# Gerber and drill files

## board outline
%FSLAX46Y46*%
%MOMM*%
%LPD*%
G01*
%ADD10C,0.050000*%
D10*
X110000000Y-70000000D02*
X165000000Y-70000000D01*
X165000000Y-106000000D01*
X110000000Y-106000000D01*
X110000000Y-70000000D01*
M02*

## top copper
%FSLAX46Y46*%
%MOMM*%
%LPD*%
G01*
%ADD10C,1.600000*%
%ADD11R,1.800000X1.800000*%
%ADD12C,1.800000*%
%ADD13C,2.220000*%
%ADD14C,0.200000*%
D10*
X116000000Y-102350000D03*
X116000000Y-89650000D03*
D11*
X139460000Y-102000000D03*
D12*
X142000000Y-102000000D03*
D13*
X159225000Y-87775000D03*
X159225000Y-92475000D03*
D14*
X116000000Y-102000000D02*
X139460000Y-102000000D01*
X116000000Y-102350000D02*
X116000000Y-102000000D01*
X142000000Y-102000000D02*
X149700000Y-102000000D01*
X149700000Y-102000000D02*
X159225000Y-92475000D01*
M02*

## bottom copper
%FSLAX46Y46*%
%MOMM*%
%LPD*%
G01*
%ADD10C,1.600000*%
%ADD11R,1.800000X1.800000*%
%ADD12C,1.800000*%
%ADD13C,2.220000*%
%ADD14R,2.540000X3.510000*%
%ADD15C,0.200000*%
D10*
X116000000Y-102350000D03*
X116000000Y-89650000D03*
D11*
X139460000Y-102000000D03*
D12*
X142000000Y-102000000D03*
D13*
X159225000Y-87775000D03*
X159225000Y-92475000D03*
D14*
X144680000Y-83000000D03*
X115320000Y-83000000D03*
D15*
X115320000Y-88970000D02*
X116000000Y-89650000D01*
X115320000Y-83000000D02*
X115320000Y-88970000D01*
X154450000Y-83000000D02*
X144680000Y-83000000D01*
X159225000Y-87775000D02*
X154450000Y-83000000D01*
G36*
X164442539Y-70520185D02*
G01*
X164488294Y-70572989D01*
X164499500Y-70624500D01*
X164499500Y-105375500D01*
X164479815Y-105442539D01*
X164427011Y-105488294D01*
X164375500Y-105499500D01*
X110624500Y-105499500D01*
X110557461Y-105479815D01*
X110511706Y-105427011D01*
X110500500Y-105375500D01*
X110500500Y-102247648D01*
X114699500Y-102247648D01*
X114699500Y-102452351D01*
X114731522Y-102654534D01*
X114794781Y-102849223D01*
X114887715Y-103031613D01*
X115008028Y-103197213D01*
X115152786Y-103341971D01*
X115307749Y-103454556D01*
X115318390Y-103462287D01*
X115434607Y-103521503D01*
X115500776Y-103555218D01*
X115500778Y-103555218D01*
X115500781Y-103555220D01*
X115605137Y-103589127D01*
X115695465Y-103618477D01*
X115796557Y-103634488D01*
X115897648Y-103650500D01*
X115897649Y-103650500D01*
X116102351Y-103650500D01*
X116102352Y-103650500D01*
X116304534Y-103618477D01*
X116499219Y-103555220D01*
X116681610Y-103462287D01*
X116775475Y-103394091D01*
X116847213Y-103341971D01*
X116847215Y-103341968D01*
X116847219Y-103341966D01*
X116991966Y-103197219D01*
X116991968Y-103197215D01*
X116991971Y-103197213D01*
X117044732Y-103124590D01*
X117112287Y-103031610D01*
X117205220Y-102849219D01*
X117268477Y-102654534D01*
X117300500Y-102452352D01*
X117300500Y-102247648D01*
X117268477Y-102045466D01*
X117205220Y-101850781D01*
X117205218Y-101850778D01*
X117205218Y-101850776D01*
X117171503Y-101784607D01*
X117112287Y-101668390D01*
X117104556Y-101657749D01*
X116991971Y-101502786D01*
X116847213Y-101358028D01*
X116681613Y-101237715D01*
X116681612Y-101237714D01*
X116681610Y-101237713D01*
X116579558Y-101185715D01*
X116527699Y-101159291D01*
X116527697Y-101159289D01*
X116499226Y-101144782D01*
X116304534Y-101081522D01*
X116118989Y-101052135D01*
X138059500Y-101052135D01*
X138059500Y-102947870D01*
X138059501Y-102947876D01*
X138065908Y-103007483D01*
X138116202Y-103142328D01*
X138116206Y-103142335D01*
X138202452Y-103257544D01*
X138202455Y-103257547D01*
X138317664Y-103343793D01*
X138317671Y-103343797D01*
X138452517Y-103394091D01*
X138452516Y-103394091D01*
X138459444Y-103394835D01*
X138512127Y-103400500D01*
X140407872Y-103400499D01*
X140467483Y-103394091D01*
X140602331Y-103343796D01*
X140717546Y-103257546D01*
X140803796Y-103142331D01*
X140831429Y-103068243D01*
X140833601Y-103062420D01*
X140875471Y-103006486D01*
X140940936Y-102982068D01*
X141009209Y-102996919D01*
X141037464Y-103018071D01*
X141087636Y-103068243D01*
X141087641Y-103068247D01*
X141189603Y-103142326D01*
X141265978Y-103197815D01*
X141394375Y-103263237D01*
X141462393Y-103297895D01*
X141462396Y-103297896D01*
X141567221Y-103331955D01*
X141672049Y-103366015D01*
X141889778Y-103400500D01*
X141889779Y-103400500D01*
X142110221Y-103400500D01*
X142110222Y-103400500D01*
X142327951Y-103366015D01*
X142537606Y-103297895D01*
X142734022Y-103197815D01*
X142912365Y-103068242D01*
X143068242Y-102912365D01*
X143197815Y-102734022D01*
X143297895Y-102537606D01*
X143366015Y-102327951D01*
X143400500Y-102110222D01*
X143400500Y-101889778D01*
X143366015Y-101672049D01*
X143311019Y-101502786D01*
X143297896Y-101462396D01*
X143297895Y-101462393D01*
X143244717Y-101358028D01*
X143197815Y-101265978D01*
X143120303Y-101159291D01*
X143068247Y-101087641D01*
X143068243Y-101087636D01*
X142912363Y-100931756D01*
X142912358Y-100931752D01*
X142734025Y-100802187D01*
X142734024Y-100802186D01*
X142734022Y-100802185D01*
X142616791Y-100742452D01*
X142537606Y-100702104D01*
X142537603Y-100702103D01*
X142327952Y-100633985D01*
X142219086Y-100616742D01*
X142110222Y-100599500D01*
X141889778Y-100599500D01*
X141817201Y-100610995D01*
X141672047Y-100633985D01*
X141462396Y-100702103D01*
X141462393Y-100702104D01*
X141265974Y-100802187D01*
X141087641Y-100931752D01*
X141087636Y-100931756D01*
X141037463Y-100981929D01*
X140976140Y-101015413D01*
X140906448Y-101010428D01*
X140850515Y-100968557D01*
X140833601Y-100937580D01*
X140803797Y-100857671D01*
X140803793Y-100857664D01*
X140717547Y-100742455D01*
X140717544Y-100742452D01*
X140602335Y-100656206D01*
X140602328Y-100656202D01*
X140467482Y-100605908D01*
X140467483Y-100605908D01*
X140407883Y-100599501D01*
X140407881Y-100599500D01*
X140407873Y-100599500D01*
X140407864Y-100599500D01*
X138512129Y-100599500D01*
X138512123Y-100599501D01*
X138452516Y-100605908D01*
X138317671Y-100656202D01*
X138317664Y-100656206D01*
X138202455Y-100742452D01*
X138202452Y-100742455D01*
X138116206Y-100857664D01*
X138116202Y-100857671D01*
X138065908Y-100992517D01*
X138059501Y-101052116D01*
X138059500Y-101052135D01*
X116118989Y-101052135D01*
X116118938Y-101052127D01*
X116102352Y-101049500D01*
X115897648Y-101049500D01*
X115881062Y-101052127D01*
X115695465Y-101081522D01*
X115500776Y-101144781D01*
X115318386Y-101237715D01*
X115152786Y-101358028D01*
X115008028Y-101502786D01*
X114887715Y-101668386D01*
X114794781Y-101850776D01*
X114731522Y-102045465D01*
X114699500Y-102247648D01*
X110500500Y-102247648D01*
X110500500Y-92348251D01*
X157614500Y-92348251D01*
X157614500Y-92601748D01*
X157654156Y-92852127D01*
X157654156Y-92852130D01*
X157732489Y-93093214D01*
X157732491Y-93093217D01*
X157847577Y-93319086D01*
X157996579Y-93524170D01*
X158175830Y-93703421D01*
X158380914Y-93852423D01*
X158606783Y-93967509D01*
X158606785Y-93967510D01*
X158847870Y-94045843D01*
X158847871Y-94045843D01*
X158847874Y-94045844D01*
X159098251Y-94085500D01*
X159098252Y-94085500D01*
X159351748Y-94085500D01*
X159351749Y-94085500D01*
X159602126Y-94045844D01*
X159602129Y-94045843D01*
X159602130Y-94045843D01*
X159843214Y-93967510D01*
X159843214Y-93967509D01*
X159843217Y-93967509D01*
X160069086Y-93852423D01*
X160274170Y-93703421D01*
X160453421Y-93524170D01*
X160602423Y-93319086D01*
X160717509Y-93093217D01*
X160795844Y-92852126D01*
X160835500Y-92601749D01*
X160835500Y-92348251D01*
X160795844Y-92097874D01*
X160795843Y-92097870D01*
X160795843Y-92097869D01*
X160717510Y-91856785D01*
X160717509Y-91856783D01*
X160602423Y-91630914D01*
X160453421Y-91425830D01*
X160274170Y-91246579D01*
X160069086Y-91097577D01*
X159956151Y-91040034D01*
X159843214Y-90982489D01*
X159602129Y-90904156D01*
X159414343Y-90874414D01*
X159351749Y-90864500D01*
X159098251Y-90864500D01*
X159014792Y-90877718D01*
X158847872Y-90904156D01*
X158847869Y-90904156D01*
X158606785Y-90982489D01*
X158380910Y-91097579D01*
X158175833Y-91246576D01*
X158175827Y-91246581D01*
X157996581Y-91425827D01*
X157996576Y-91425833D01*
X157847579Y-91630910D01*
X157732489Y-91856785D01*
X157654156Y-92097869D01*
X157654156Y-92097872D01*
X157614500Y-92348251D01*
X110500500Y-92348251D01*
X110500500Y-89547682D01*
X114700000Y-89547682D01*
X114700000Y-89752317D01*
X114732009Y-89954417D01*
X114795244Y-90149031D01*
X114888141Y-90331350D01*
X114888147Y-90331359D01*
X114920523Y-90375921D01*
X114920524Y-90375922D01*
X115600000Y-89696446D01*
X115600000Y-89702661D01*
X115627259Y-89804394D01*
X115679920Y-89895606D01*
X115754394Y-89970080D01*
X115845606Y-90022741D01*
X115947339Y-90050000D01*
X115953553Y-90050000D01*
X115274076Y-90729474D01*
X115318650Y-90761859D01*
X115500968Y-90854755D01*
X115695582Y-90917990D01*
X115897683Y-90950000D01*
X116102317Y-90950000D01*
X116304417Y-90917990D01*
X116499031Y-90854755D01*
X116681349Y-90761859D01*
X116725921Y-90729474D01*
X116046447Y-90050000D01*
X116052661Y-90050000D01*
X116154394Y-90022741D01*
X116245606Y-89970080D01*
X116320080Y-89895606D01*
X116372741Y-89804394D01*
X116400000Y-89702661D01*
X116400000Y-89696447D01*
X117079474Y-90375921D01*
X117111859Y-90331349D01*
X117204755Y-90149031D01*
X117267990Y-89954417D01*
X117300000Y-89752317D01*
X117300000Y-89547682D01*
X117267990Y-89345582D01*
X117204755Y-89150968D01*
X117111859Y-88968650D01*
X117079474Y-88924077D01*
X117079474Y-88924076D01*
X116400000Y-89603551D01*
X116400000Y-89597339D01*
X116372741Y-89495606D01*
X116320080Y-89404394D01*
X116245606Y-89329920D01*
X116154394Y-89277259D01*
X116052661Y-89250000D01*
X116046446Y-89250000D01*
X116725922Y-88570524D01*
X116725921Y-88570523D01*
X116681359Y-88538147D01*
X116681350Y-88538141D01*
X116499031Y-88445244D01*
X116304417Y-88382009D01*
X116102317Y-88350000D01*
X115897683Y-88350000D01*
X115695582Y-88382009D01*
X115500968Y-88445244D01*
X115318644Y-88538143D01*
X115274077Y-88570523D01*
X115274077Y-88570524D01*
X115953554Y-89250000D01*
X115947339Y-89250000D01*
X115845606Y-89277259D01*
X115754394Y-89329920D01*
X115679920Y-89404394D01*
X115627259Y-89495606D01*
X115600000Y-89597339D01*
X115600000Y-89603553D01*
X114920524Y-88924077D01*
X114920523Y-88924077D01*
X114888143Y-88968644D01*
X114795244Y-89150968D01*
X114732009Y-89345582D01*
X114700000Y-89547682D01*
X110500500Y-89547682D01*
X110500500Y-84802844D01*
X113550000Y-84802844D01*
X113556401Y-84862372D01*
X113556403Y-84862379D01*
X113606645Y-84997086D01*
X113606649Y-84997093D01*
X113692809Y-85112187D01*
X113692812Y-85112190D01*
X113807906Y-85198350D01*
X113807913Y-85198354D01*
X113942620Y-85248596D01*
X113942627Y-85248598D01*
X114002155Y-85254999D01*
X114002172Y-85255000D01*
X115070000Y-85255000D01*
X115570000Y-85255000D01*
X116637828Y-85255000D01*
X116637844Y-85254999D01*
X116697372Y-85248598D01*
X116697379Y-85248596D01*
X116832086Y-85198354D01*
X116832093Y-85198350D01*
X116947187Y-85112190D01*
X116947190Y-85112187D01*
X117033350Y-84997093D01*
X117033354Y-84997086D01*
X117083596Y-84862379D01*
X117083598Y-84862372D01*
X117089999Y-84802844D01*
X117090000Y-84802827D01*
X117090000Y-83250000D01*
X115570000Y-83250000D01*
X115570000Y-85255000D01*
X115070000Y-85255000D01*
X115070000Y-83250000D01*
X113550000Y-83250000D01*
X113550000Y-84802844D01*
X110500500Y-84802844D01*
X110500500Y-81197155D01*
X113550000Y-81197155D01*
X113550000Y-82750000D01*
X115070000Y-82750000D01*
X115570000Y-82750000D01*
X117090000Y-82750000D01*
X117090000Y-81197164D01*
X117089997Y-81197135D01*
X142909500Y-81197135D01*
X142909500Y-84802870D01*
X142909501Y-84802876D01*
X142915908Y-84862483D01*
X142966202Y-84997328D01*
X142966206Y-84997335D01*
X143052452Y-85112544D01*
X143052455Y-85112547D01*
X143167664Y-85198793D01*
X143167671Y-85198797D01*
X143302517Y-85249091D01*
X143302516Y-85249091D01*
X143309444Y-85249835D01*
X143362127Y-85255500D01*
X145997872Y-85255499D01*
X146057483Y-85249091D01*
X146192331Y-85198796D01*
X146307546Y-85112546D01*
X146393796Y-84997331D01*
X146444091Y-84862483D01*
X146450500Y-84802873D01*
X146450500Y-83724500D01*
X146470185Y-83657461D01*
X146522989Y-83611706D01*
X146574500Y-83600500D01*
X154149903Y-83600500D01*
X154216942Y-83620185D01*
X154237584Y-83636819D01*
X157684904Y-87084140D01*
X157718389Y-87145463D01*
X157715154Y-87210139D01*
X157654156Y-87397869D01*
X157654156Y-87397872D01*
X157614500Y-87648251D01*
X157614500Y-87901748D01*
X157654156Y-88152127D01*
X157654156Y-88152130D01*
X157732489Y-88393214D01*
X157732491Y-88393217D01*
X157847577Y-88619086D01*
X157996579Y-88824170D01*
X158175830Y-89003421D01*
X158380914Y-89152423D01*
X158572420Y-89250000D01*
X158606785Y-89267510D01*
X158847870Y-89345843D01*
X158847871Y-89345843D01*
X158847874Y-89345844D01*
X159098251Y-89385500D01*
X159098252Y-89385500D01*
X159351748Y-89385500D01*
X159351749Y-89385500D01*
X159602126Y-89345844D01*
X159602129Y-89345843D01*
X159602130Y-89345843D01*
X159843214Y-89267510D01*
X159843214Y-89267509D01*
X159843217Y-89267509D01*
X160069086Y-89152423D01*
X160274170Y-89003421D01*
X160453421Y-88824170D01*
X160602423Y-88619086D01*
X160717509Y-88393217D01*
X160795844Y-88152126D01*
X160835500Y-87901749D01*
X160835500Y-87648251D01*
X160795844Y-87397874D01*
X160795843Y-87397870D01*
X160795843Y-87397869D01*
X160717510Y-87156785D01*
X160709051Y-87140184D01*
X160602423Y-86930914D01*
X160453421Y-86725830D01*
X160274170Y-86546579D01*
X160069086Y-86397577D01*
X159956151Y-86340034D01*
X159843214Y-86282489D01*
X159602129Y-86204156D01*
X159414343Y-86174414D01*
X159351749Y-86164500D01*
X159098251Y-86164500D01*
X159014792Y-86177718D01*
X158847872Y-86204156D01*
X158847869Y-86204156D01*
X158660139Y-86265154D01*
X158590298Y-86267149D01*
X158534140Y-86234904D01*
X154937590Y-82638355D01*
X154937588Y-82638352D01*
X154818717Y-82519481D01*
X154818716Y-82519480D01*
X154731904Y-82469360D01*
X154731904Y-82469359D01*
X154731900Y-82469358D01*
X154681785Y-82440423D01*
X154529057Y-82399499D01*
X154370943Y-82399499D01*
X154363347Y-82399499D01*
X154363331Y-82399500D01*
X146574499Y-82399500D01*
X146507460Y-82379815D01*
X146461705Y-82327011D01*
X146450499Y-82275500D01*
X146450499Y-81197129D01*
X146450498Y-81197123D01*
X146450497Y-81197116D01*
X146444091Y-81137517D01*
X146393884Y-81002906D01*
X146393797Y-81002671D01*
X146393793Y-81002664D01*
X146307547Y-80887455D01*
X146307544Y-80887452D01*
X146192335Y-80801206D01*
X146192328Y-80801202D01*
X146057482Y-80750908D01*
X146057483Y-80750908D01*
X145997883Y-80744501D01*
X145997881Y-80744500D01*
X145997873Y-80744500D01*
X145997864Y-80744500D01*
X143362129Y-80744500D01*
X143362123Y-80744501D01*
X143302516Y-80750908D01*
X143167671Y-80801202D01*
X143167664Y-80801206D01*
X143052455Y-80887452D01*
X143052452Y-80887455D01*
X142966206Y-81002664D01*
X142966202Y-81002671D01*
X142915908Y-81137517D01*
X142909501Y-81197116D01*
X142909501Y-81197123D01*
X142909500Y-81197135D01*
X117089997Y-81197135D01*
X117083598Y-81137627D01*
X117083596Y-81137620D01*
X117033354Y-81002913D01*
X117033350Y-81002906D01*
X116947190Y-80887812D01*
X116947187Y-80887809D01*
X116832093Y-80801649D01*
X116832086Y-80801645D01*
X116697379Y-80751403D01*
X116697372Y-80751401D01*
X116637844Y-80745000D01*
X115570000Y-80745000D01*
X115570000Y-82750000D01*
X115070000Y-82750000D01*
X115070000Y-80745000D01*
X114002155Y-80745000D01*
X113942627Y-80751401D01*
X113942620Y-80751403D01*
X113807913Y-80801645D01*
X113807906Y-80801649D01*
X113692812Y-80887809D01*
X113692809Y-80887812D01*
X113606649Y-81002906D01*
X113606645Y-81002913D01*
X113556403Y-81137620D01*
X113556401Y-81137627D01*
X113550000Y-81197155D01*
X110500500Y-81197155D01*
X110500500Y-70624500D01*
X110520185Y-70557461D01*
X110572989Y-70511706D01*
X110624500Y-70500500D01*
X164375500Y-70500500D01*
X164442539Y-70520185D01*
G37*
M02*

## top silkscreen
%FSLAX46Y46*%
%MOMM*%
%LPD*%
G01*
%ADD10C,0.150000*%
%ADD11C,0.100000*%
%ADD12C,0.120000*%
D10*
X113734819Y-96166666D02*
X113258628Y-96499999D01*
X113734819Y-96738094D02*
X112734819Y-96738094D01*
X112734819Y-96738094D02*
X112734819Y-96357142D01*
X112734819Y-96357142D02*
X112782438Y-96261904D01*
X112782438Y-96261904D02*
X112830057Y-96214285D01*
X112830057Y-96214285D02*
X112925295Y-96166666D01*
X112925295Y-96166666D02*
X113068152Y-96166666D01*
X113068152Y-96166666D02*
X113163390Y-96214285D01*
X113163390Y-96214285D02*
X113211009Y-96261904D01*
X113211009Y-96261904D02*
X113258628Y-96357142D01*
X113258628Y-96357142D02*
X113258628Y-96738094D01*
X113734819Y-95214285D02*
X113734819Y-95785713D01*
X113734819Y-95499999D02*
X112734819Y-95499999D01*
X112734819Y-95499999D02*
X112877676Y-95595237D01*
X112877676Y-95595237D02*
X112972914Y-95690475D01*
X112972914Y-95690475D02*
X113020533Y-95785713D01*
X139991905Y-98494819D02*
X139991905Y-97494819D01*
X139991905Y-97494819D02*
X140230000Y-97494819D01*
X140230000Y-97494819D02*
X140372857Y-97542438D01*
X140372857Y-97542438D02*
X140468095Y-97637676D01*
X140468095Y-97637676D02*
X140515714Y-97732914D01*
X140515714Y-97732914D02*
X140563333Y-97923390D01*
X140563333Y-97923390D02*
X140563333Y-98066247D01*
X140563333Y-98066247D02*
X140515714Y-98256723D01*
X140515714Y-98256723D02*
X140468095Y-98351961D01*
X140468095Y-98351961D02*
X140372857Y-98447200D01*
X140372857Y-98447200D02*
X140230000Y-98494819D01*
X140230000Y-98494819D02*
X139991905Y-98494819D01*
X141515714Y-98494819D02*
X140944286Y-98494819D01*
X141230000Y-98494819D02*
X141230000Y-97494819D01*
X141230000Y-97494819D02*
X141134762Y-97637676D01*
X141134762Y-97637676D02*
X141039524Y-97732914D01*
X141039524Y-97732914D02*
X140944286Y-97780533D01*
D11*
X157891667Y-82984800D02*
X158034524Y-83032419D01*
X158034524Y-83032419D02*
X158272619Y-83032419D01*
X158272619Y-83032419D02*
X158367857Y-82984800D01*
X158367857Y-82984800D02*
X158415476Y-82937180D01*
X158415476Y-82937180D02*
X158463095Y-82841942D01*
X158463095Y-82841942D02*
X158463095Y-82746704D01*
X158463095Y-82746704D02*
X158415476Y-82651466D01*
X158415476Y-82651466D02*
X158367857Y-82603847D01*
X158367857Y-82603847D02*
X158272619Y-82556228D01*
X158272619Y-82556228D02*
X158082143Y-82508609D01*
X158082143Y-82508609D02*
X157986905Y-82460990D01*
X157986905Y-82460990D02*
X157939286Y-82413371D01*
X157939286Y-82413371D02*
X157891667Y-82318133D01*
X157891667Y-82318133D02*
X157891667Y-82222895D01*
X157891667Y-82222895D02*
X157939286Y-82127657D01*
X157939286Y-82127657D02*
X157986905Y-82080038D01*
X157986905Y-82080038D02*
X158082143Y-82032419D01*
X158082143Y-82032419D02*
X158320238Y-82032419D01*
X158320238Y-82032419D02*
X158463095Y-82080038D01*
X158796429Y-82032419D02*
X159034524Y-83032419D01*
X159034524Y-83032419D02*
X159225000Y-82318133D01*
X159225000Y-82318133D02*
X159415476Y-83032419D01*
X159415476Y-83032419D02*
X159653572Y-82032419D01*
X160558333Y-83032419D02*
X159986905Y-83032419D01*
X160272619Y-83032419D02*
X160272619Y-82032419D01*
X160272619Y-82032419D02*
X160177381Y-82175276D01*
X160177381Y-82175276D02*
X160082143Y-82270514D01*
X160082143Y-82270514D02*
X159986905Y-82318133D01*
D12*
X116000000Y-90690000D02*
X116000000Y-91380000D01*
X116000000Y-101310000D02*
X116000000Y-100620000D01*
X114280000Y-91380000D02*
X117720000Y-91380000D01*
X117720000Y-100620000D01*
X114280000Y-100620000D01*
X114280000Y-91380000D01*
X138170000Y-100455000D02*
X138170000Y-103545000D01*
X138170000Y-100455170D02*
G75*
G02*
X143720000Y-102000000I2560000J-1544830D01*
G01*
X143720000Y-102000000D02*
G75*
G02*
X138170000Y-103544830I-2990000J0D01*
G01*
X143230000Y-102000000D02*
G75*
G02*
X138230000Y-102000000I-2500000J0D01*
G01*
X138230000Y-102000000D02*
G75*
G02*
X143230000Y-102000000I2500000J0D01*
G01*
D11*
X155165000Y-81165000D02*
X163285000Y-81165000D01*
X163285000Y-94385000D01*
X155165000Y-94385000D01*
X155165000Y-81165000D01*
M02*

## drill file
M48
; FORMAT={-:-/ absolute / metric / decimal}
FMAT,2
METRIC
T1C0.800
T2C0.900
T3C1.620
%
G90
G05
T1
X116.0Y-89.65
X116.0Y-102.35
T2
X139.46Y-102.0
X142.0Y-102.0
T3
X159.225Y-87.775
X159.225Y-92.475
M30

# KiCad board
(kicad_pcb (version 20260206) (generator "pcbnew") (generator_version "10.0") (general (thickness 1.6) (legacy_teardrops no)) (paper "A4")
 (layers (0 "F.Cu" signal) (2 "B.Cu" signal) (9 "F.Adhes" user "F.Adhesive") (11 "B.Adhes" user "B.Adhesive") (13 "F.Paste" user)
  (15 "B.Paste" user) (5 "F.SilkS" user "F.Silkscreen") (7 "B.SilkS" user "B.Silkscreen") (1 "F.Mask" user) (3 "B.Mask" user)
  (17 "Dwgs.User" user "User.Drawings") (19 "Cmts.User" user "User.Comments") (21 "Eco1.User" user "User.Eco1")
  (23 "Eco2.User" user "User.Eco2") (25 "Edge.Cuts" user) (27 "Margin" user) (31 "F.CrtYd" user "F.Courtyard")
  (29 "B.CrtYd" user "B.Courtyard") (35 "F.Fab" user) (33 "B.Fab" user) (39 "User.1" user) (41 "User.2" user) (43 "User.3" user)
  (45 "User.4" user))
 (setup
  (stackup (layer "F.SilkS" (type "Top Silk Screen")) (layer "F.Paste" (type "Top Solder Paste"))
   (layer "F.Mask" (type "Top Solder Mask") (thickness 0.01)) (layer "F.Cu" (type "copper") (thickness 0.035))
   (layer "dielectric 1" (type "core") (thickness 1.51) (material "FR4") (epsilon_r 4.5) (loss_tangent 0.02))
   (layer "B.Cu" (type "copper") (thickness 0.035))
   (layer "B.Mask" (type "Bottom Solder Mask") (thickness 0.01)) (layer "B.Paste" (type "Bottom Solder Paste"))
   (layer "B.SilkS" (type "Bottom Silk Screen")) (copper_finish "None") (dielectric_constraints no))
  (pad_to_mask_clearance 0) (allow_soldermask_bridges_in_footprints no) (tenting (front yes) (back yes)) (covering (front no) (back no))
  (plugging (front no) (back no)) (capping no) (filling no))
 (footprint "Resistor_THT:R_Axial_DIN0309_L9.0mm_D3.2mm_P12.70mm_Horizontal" (layer "F.Cu") (at 116 102.35 90)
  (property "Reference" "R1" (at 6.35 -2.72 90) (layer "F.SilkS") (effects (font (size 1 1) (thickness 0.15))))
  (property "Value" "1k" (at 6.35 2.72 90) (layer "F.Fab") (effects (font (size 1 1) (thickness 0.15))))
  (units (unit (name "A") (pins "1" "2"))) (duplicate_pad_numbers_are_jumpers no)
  (fp_line (start 11.66 0) (end 10.97 0) (stroke (width 0.12) (type solid)) (layer "F.SilkS"))
  (fp_line (start 1.04 0) (end 1.73 0) (stroke (width 0.12) (type solid)) (layer "F.SilkS"))
  (fp_rect (start 1.73 -1.72) (end 10.97 1.72) (stroke (width 0.12) (type solid)) (fill no) (layer "F.SilkS"))
  (pad "1" thru_hole circle (at 0 0 90) (size 1.6 1.6) (drill 0.8) (layers "*.Cu" "*.Mask") (remove_unused_layers no) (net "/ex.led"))
  (pad "2" thru_hole circle (at 12.7 0 90) (size 1.6 1.6) (drill 0.8) (layers "*.Cu" "*.Mask") (remove_unused_layers no) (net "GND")))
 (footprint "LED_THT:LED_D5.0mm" (layer "F.Cu") (at 139.46 102)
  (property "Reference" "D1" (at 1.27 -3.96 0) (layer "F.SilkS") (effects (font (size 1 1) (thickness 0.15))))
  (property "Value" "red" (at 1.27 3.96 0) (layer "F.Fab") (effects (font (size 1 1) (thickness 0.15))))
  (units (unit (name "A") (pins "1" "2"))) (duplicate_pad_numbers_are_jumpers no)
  (fp_line (start -1.29 -1.545) (end -1.29 1.545) (stroke (width 0.12) (type solid)) (layer "F.SilkS"))
  (fp_arc (start -1.29 -1.54483) (mid 2.071779 -2.880495) (end 4.26 0) (stroke (width 0.12) (type solid)) (layer "F.SilkS"))
  (fp_arc (start 4.26 0) (mid 2.071779 2.880495) (end -1.29 1.54483) (stroke (width 0.12) (type solid)) (layer "F.SilkS"))
  (fp_circle (center 1.27 0) (end 3.77 0) (stroke (width 0.12) (type solid)) (fill no) (layer "F.SilkS"))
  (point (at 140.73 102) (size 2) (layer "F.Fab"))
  (pad "1" thru_hole rect (at 0 0) (size 1.8 1.8) (drill 0.9) (layers "*.Cu" "*.Mask") (remove_unused_layers no) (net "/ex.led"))
  (pad "2" thru_hole circle (at 2.54 0) (size 1.8 1.8) (drill 0.9) (layers "*.Cu" "*.Mask") (remove_unused_layers no) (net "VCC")))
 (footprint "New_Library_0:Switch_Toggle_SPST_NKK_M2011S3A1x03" (layer "F.Cu") (at 159.225 83.075)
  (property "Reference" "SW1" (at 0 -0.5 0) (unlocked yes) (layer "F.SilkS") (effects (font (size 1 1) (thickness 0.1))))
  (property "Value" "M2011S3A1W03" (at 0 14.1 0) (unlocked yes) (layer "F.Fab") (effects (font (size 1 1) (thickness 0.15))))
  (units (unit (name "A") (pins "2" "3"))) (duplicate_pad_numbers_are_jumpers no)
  (fp_rect (start -4.06 -1.91) (end 4.06 11.31) (stroke (width 0.1) (type solid)) (fill no) (layer "F.SilkS"))
  (pad "2" thru_hole circle (at 0 4.7) (size 2.22 2.22) (drill 1.62) (layers "*.Cu" "*.Mask") (remove_unused_layers no) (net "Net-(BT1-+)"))
  (pad "3" thru_hole circle (at 0 9.4) (size 2.22 2.22) (drill 1.62) (layers "*.Cu" "*.Mask") (remove_unused_layers no) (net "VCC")))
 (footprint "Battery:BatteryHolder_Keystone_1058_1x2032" (layer "B.Cu") (at 130 83 180)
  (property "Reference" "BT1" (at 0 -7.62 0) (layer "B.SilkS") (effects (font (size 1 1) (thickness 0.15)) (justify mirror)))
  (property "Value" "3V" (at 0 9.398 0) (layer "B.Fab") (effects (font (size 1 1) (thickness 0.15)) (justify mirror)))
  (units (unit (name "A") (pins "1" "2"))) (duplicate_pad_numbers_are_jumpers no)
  (pad "1" smd rect (at -14.68 0 180) (size 2.54 3.51) (layers "B.Cu" "B.Mask" "B.Paste") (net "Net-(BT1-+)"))
  (pad "2" smd rect (at 14.68 0 180) (size 2.54 3.51) (layers "B.Cu" "B.Mask" "B.Paste") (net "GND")))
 (gr_rect (start 110 70) (end 165 106) (stroke (width 0.05) (type default)) (fill no) (layer "Edge.Cuts"))
 (segment (start 116 102) (end 139.46 102) (width 0.2) (layer "F.Cu") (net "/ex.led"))
 (segment (start 116 102.35) (end 116 102) (width 0.2) (layer "F.Cu") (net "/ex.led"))
 (segment (start 115.32 88.97) (end 116 89.65) (width 0.2) (layer "B.Cu") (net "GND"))
 (segment (start 115.32 83) (end 115.32 88.97) (width 0.2) (layer "B.Cu") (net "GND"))
 (segment (start 142 102) (end 149.7 102) (width 0.2) (layer "F.Cu") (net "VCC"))
 (segment (start 149.7 102) (end 159.225 92.475) (width 0.2) (layer "F.Cu") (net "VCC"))
 (segment (start 154.45 83) (end 144.68 83) (width 0.2) (layer "B.Cu") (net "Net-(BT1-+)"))
 (segment (start 159.225 87.775) (end 154.45 83) (width 0.2) (layer "B.Cu") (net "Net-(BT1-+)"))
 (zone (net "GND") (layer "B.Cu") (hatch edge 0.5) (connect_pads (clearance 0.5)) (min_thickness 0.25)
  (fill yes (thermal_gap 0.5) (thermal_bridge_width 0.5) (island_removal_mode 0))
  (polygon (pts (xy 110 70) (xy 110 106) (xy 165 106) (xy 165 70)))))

